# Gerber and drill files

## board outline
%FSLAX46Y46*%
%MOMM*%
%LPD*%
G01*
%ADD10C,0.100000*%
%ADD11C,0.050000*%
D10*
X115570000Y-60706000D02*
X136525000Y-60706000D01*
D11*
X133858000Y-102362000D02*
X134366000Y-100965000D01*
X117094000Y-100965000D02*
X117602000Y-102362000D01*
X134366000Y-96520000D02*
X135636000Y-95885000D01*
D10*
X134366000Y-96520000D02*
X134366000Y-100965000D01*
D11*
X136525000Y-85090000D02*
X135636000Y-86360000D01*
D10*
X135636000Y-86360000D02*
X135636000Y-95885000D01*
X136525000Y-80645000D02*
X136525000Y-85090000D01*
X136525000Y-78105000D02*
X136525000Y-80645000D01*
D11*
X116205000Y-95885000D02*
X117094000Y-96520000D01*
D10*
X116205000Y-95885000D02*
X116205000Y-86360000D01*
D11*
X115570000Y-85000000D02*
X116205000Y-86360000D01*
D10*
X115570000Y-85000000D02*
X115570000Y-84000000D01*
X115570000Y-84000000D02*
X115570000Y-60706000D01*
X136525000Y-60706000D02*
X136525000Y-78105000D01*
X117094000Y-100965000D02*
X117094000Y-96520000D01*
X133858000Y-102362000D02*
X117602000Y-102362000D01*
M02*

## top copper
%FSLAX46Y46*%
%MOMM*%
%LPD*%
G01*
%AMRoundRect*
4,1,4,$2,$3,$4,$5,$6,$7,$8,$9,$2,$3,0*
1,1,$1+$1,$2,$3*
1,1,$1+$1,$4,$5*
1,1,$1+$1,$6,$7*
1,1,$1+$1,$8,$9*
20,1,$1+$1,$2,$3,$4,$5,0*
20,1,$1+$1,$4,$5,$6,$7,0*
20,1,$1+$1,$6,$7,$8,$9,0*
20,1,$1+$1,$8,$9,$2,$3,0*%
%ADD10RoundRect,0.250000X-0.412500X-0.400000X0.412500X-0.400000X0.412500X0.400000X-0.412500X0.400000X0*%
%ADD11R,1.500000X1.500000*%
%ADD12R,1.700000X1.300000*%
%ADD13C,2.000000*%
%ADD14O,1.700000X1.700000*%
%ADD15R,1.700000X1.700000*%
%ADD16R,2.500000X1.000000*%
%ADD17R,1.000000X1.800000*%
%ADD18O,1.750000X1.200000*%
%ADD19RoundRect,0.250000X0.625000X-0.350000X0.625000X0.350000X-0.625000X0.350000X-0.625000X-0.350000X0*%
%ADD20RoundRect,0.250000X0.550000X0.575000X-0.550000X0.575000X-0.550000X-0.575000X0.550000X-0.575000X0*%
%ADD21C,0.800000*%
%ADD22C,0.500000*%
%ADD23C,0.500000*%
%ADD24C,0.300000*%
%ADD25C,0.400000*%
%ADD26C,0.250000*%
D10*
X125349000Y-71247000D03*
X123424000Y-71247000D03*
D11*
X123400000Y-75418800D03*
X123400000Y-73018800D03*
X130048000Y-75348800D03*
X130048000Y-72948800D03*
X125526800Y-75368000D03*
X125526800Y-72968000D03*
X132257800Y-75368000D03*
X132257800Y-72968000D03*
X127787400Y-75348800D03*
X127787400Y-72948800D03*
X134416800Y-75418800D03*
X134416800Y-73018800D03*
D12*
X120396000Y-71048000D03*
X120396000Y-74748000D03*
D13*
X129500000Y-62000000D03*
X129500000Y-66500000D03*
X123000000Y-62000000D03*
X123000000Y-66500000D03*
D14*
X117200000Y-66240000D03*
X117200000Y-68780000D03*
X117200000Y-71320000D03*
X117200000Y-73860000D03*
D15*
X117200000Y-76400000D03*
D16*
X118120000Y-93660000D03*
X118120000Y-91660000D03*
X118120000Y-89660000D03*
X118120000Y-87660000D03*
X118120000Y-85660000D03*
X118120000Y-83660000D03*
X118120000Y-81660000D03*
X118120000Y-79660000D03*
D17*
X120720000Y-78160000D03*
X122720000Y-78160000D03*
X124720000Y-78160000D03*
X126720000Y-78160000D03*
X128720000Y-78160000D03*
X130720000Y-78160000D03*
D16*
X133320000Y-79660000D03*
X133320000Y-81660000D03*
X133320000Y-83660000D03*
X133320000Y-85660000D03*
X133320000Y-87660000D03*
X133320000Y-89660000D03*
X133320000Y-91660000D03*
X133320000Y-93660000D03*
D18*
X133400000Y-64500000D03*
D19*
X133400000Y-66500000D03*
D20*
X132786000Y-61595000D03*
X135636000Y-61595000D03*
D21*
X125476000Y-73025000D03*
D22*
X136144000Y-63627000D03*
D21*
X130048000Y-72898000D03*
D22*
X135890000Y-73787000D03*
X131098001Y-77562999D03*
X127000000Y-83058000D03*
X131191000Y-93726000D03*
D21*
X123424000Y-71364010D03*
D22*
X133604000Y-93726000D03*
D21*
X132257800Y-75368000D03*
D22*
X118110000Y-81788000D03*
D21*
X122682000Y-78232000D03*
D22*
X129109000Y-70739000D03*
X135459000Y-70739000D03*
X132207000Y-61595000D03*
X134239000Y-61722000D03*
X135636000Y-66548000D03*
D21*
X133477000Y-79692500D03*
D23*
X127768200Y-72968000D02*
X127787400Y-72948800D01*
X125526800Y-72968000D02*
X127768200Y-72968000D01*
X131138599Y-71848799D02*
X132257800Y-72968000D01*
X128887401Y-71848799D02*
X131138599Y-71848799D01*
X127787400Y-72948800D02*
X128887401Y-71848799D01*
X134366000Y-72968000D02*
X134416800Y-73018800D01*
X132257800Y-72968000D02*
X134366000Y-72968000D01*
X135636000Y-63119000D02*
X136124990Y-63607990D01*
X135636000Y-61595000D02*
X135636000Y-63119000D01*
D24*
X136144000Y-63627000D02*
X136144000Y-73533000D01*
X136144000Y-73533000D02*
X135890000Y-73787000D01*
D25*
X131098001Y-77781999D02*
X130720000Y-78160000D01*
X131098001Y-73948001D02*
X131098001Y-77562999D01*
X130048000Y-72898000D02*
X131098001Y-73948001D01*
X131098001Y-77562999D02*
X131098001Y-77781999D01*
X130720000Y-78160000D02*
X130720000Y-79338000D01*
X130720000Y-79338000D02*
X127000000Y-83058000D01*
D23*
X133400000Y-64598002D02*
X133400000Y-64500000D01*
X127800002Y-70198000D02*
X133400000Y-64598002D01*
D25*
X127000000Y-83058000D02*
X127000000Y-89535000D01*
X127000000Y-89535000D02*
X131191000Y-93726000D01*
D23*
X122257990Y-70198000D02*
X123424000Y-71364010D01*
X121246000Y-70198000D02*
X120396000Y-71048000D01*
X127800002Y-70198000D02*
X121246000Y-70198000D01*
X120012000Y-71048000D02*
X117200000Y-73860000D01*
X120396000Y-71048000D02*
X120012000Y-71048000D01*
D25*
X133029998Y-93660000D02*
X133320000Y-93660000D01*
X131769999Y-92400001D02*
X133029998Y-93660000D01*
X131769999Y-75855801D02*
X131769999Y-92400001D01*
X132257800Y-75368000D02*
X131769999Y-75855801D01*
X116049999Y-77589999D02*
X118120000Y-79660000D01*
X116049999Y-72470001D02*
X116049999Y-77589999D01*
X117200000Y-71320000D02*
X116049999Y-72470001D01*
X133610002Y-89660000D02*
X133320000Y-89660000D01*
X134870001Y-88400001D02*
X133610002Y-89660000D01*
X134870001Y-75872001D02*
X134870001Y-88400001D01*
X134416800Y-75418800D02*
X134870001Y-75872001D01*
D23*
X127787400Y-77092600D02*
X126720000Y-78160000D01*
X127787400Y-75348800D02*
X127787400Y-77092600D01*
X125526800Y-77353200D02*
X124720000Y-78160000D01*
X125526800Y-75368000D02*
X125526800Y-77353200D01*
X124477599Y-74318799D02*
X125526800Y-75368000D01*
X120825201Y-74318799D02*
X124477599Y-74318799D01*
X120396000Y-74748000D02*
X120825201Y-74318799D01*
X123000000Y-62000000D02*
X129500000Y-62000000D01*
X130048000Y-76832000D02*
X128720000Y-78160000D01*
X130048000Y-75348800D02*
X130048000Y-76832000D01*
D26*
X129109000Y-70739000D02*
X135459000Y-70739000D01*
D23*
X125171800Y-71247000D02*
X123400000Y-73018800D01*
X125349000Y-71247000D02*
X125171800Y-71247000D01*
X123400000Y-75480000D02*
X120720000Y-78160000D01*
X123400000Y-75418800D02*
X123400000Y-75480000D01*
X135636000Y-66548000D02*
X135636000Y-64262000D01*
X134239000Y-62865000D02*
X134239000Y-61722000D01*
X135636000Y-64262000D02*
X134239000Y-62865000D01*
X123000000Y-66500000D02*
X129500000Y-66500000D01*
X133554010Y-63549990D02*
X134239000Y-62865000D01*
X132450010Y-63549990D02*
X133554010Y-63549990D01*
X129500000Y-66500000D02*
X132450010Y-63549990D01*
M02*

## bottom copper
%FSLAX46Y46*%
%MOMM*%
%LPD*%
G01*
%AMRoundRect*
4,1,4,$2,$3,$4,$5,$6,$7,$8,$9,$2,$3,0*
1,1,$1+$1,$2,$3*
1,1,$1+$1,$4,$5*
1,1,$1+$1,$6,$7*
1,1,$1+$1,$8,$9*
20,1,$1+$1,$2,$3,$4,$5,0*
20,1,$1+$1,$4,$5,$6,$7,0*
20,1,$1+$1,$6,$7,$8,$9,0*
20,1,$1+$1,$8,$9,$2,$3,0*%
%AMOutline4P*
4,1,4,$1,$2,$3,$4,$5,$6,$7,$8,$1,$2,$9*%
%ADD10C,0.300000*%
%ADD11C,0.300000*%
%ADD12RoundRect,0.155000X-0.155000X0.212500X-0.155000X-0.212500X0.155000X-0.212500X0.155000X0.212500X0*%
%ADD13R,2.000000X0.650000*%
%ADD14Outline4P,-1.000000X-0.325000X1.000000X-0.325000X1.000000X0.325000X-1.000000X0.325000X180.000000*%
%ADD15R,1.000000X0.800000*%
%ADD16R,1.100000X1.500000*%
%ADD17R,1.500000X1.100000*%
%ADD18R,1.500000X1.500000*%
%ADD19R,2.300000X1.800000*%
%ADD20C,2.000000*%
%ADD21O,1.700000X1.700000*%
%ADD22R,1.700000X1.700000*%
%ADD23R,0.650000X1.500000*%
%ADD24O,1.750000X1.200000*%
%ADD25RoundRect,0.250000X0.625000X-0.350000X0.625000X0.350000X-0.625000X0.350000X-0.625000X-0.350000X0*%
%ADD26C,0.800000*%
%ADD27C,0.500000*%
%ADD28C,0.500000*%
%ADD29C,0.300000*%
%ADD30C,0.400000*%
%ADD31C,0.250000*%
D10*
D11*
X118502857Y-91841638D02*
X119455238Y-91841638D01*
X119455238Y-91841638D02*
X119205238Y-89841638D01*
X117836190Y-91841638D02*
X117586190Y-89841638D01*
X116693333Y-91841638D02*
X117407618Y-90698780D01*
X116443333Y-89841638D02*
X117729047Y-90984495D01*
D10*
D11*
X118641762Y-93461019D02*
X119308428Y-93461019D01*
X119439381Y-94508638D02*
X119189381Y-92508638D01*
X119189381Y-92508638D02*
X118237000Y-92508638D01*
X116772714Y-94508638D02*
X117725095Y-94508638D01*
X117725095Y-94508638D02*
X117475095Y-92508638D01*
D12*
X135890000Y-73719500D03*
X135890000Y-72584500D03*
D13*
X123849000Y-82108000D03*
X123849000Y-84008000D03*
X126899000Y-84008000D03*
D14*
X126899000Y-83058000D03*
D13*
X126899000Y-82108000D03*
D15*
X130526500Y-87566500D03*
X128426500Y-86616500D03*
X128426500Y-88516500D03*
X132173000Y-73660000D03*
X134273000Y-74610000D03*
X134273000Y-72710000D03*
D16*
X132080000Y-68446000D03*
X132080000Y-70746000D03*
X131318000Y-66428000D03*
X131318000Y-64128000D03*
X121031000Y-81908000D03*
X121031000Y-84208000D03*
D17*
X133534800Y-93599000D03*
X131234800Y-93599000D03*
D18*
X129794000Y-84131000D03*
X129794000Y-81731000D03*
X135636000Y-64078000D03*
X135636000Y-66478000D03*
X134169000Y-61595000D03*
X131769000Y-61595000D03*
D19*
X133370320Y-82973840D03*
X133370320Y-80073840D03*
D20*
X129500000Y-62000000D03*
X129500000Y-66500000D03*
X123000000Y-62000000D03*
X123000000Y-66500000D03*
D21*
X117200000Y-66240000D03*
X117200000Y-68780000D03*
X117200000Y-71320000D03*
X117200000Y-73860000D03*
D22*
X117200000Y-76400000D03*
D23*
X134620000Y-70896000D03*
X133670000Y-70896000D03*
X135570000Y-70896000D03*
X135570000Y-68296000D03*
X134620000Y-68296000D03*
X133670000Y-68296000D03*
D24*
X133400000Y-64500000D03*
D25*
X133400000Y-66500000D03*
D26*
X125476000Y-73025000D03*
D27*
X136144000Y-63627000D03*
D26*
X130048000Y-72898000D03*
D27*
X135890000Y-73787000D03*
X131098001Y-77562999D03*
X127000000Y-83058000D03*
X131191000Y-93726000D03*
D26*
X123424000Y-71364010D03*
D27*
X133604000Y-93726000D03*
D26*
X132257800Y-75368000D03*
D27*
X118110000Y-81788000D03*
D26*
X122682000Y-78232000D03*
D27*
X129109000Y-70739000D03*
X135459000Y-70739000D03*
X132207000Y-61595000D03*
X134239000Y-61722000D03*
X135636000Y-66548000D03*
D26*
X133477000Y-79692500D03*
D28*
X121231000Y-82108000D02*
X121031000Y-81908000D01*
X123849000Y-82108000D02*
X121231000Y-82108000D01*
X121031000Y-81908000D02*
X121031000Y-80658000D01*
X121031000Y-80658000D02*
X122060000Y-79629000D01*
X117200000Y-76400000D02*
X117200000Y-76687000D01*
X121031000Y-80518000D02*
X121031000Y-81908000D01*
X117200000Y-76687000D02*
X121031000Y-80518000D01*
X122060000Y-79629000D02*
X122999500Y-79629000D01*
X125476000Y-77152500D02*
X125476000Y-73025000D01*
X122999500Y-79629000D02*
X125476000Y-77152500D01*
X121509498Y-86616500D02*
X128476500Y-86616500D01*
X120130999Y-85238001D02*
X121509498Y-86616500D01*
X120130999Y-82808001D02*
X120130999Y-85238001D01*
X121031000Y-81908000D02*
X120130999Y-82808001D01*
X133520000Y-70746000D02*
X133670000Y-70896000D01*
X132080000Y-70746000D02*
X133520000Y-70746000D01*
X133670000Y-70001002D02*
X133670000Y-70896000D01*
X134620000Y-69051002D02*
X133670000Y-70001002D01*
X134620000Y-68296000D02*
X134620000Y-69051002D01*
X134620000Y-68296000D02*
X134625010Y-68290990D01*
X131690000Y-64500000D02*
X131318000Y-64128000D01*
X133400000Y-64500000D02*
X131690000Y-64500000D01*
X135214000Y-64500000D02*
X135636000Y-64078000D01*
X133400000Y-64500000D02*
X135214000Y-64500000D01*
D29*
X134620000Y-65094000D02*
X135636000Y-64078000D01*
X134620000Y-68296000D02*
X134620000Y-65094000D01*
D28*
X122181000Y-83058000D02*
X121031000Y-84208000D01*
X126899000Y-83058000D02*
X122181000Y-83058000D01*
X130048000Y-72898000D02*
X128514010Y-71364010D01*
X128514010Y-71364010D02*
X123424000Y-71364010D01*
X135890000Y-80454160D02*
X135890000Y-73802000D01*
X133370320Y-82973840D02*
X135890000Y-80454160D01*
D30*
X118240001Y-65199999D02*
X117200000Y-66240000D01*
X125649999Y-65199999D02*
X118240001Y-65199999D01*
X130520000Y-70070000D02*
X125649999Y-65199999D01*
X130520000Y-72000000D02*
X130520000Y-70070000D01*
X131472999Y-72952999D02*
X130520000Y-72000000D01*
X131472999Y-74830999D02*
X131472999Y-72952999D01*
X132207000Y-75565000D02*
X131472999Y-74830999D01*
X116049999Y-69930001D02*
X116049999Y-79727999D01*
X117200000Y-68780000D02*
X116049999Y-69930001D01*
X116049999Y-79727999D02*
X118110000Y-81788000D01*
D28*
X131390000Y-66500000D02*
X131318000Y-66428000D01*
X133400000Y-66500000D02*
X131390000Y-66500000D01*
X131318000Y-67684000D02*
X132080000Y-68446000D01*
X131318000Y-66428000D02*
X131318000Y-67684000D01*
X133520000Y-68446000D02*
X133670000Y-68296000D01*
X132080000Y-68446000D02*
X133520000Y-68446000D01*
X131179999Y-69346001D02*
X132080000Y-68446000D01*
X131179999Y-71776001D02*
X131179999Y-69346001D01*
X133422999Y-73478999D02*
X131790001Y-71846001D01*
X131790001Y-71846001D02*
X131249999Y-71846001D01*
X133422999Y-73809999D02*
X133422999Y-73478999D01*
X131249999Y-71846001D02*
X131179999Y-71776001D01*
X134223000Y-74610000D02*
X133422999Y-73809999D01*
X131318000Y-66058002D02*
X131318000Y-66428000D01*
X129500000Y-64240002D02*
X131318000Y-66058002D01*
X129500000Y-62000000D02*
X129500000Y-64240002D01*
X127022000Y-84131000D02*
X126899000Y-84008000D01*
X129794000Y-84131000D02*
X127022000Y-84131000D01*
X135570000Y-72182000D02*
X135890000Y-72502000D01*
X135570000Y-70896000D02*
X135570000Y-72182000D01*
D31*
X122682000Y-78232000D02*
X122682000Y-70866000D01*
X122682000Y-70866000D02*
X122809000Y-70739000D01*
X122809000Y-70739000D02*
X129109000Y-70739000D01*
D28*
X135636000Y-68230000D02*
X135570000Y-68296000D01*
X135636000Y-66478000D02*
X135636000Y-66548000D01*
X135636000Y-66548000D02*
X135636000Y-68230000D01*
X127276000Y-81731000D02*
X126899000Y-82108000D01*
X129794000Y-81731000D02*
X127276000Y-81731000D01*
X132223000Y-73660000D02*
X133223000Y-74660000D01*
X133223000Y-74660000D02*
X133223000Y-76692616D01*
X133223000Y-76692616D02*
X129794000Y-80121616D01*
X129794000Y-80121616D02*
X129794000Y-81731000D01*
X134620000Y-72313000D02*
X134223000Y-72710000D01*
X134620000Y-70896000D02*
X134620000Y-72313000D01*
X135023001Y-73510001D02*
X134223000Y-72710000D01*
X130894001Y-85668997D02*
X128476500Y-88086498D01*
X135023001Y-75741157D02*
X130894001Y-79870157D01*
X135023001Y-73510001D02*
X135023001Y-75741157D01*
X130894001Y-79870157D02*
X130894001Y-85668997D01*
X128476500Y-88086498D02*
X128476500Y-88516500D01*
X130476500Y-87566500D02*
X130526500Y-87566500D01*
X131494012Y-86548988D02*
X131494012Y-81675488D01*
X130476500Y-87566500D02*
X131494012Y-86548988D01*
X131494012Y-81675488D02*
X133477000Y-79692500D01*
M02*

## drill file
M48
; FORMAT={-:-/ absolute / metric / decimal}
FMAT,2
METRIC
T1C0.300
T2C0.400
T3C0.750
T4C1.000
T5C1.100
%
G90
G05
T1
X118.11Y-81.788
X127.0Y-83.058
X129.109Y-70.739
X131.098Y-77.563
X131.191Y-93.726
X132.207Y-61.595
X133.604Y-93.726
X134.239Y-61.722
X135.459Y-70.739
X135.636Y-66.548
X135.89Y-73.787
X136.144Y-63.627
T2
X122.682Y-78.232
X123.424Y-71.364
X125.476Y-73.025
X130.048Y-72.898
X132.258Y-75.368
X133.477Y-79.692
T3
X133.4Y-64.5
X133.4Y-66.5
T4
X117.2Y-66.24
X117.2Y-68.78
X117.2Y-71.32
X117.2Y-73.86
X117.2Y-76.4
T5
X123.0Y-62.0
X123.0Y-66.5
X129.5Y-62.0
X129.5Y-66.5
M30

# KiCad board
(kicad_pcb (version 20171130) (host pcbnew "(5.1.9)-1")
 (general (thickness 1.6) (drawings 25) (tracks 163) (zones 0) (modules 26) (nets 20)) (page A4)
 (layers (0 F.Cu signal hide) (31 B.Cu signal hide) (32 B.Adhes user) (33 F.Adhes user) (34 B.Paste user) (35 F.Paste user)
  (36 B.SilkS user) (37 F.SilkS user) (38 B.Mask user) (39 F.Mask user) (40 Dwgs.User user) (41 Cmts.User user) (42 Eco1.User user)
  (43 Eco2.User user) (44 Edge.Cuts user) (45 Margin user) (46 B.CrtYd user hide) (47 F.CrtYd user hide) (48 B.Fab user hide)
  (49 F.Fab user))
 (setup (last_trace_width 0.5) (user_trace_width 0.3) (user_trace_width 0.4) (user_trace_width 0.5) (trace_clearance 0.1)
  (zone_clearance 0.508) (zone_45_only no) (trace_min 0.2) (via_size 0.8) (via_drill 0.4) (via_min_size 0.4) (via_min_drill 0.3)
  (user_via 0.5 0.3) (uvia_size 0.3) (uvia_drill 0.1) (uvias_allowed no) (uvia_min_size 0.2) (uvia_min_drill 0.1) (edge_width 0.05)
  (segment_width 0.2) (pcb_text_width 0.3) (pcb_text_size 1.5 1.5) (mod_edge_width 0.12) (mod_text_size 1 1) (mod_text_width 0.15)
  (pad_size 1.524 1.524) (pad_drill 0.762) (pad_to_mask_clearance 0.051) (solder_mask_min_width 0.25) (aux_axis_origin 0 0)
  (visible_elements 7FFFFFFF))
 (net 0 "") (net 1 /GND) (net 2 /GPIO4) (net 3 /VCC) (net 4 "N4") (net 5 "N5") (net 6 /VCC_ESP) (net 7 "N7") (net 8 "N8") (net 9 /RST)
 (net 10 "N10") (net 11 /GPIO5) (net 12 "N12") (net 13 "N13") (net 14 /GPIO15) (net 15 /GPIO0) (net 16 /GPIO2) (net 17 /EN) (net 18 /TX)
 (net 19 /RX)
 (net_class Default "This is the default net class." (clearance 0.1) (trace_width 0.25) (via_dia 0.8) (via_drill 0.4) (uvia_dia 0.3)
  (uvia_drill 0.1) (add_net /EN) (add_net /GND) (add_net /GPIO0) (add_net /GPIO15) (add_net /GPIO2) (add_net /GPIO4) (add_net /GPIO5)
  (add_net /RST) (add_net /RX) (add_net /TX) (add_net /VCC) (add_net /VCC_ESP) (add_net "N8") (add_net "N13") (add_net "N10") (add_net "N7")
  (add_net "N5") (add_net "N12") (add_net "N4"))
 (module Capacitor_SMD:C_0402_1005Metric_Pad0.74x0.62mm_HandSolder (layer B.Cu) (at 135.89 73.152 270)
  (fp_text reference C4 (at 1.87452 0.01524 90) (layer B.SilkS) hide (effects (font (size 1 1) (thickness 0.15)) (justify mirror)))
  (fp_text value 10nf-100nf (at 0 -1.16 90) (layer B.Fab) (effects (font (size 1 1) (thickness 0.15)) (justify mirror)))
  (pad 2 smd roundrect (at 0.5675 0 270) (size 0.735 0.62) (layers B.Cu B.Paste B.Mask) (roundrect_rratio 0.25) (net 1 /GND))
  (pad 1 smd roundrect (at -0.5675 0 270) (size 0.735 0.62) (layers B.Cu B.Paste B.Mask) (roundrect_rratio 0.25) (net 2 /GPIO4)))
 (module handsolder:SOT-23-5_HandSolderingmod (layer B.Cu) (at 125.349 83.058 180)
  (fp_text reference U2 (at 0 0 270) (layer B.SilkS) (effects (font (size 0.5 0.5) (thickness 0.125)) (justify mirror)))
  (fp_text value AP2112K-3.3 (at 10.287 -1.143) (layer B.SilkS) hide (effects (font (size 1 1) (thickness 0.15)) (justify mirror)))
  (pad 5 smd rect (at 1.5 0.95 180) (size 2 0.65) (layers B.Cu B.Paste B.Mask) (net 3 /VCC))
  (pad 4 smd rect (at 1.5 -0.95 180) (size 2 0.65) (layers B.Cu B.Paste B.Mask))
  (pad 3 smd rect (at -1.55 -0.95 180) (size 2 0.65) (layers B.Cu B.Paste B.Mask) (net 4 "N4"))
  (pad 2 smd trapezoid (at -1.55 0 180) (size 2 0.65) (layers B.Cu B.Paste B.Mask) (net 1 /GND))
  (pad 1 smd rect (at -1.55 0.95 180) (size 2 0.65) (layers B.Cu B.Paste B.Mask) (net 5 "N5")))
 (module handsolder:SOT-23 (layer B.Cu) (at 129.4765 87.5665)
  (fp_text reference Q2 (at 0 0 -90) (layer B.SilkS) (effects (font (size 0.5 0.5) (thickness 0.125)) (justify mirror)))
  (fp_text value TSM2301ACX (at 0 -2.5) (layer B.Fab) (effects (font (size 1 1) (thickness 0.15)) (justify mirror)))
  (pad 3 smd rect (at 1.05 0) (size 1 0.8) (layers B.Cu B.Paste B.Mask) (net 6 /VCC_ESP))
  (pad 2 smd rect (at -1.05 -0.95) (size 1 0.8) (layers B.Cu B.Paste B.Mask) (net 3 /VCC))
  (pad 1 smd rect (at -1.05 0.95) (size 1 0.8) (layers B.Cu B.Paste B.Mask) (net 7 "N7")))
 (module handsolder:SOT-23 (layer B.Cu) (at 133.223 73.66 180)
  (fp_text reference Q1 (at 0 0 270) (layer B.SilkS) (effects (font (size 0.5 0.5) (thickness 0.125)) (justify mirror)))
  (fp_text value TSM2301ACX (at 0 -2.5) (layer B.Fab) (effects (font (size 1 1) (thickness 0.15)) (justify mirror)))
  (pad 3 smd rect (at 1.05 0 180) (size 1 0.8) (layers B.Cu B.Paste B.Mask) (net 5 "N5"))
  (pad 2 smd rect (at -1.05 -0.95 180) (size 1 0.8) (layers B.Cu B.Paste B.Mask) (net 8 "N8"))
  (pad 1 smd rect (at -1.05 0.95 180) (size 1 0.8) (layers B.Cu B.Paste B.Mask) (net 7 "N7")))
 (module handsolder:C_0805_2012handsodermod (layer B.Cu) (at 132.08 69.596 90)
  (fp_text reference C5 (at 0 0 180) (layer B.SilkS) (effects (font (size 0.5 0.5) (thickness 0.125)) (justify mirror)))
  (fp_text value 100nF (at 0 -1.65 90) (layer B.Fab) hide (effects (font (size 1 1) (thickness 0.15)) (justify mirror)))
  (pad 2 smd rect (at 1.15 0 90) (size 1.5 1.1) (layers B.Cu B.Paste B.Mask) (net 8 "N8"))
  (pad 1 smd rect (at -1.15 0 90) (size 1.5 1.1) (layers B.Cu B.Paste B.Mask) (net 1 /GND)))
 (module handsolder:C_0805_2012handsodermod (layer B.Cu) (at 131.318 65.278 270)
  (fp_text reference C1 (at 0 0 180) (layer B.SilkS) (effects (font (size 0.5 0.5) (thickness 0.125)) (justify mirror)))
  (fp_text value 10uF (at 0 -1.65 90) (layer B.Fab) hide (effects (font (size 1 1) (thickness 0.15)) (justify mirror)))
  (pad 2 smd rect (at 1.15 0 270) (size 1.5 1.1) (layers B.Cu B.Paste B.Mask) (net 8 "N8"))
  (pad 1 smd rect (at -1.15 0 270) (size 1.5 1.1) (layers B.Cu B.Paste B.Mask) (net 1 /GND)))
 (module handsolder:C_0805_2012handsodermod (layer B.Cu) (at 121.031 83.058 90)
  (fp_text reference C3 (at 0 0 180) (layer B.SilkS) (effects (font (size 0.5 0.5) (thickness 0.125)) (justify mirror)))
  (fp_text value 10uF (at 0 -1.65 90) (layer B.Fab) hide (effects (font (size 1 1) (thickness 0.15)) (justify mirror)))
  (pad 2 smd rect (at 1.15 0 90) (size 1.5 1.1) (layers B.Cu B.Paste B.Mask) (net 3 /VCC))
  (pad 1 smd rect (at -1.15 0 90) (size 1.5 1.1) (layers B.Cu B.Paste B.Mask) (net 1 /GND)))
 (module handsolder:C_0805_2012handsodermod (layer B.Cu) (at 132.3848 93.599)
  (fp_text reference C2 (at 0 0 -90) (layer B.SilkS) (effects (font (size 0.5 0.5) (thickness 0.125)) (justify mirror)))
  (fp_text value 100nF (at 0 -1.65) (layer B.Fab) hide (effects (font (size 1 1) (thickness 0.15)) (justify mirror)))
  (pad 2 smd rect (at 1.15 0) (size 1.5 1.1) (layers B.Cu B.Paste B.Mask) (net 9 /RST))
  (pad 1 smd rect (at -1.15 0) (size 1.5 1.1) (layers B.Cu B.Paste B.Mask) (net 1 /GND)))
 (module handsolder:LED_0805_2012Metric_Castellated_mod (layer F.Cu) (at 124.3865 71.247)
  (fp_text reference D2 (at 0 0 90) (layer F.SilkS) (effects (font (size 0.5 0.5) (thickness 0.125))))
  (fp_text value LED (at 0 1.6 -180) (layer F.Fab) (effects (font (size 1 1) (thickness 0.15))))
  (pad 2 smd roundrect (at 0.9625 0) (size 1.325 1.3) (layers F.Cu F.Paste F.Mask) (roundrect_rratio 0.1923076923076923) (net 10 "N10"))
  (pad 1 smd roundrect (at -0.9625 0) (size 1.325 1.3) (layers F.Cu F.Paste F.Mask) (roundrect_rratio 0.1923076923076923) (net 1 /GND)))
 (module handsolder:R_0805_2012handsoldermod (layer F.Cu) (at 123.4 74.2188 270)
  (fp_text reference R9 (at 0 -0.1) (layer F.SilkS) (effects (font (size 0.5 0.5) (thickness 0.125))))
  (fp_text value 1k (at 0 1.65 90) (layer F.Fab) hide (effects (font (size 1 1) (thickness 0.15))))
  (pad 2 smd rect (at 1.2 0 270) (size 1.5 1.5) (layers F.Cu F.Paste F.Mask) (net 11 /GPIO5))
  (pad 1 smd rect (at -1.2 0 270) (size 1.5 1.5) (layers F.Cu F.Paste F.Mask) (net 10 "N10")))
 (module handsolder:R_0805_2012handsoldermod (layer B.Cu) (at 129.794 82.931 270)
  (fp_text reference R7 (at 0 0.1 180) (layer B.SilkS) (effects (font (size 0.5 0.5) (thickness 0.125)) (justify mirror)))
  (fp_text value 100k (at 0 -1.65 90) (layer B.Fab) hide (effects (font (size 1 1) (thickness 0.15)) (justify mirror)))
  (pad 2 smd rect (at 1.2 0 270) (size 1.5 1.5) (layers B.Cu B.Paste B.Mask) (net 4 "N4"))
  (pad 1 smd rect (at -1.2 0 270) (size 1.5 1.5) (layers B.Cu B.Paste B.Mask) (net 5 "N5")))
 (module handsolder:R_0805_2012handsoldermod (layer B.Cu) (at 135.636 65.278 90)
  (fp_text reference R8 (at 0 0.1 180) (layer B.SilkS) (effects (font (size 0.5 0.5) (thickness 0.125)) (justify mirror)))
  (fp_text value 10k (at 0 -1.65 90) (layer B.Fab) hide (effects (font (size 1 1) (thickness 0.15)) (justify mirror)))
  (pad 2 smd rect (at 1.2 0 90) (size 1.5 1.5) (layers B.Cu B.Paste B.Mask) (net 1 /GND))
  (pad 1 smd rect (at -1.2 0 90) (size 1.5 1.5) (layers B.Cu B.Paste B.Mask) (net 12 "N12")))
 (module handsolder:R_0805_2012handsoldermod (layer B.Cu) (at 132.969 61.595)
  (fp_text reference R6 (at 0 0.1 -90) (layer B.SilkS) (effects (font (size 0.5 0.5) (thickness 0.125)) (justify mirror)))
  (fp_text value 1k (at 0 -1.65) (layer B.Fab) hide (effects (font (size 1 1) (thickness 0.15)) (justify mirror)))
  (pad 2 smd rect (at 1.2 0) (size 1.5 1.5) (layers B.Cu B.Paste B.Mask) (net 12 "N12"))
  (pad 1 smd rect (at -1.2 0) (size 1.5 1.5) (layers B.Cu B.Paste B.Mask) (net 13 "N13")))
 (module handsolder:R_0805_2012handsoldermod (layer F.Cu) (at 130.048 74.1488 270)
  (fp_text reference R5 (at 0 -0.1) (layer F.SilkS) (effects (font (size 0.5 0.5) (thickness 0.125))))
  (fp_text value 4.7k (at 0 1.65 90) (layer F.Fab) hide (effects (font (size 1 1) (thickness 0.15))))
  (pad 2 smd rect (at 1.2 0 270) (size 1.5 1.5) (layers F.Cu F.Paste F.Mask) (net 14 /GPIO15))
  (pad 1 smd rect (at -1.2 0 270) (size 1.5 1.5) (layers F.Cu F.Paste F.Mask) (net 1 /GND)))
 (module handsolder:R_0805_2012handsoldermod (layer F.Cu) (at 125.5268 74.168 270)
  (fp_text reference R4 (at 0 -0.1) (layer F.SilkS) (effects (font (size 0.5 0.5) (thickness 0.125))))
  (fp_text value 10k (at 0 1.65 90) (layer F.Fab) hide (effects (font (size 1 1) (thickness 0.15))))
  (pad 2 smd rect (at 1.2 0 270) (size 1.5 1.5) (layers F.Cu F.Paste F.Mask) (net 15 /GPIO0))
  (pad 1 smd rect (at -1.2 0 270) (size 1.5 1.5) (layers F.Cu F.Paste F.Mask) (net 3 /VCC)))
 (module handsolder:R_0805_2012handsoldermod (layer F.Cu) (at 132.2578 74.168 270)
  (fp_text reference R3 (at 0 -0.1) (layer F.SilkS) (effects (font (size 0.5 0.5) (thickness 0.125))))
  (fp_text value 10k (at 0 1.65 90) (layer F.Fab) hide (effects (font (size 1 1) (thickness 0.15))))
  (pad 2 smd rect (at 1.2 0 270) (size 1.5 1.5) (layers F.Cu F.Paste F.Mask) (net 9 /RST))
  (pad 1 smd rect (at -1.2 0 270) (size 1.5 1.5) (layers F.Cu F.Paste F.Mask) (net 3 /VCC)))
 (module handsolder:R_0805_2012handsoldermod (layer F.Cu) (at 127.7874 74.1488 270)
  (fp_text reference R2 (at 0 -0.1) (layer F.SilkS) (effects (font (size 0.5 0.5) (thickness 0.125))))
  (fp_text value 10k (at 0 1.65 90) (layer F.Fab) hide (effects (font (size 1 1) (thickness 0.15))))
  (pad 2 smd rect (at 1.2 0 270) (size 1.5 1.5) (layers F.Cu F.Paste F.Mask) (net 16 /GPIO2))
  (pad 1 smd rect (at -1.2 0 270) (size 1.5 1.5) (layers F.Cu F.Paste F.Mask) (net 3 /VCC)))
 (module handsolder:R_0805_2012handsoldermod (layer F.Cu) (at 134.4168 74.2188 270)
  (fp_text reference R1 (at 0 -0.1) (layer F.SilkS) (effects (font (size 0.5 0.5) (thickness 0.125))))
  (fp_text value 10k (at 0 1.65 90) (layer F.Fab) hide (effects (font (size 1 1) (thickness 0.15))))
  (pad 2 smd rect (at 1.2 0 270) (size 1.5 1.5) (layers F.Cu F.Paste F.Mask) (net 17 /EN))
  (pad 1 smd rect (at -1.2 0 270) (size 1.5 1.5) (layers F.Cu F.Paste F.Mask) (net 3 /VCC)))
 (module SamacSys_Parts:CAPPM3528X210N (layer B.Cu) (at 133.37032 81.52384 270)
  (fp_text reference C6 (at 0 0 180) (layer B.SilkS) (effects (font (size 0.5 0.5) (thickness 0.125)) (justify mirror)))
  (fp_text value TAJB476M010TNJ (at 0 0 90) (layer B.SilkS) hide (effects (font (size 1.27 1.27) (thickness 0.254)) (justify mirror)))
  (pad 2 smd rect (at 1.45 0 270) (size 1.8 2.3) (layers B.Cu B.Paste B.Mask) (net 1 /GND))
  (pad 1 smd rect (at -1.45 0 270) (size 1.8 2.3) (layers B.Cu B.Paste B.Mask) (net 6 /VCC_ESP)))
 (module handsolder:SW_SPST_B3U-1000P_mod (layer F.Cu) (at 120.396 72.898 90)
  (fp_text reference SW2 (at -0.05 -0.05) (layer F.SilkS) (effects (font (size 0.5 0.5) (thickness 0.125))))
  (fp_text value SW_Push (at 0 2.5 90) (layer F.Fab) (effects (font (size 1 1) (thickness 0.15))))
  (pad 2 smd rect (at 1.85 0 90) (size 1.3 1.7) (layers F.Cu F.Paste F.Mask) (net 1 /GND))
  (pad 1 smd rect (at -1.85 0 90) (size 1.3 1.7) (layers F.Cu F.Paste F.Mask) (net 15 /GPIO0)))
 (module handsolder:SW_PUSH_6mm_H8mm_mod (layer F.Cu) (at 123 62)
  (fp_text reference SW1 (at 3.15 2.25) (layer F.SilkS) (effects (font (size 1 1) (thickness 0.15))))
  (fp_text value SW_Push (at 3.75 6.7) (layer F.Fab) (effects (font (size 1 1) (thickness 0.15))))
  (pad 1 thru_hole circle (at 6.5 0 90) (size 2 2) (drill 1.1) (layers *.Cu *.Mask) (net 8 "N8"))
  (pad 2 thru_hole circle (at 6.5 4.5 90) (size 2 2) (drill 1.1) (layers *.Cu *.Mask) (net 12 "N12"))
  (pad 1 thru_hole circle (at 0 0 90) (size 2 2) (drill 1.1) (layers *.Cu *.Mask) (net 8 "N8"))
  (pad 2 thru_hole circle (at 0 4.5 90) (size 2 2) (drill 1.1) (layers *.Cu *.Mask) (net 12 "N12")))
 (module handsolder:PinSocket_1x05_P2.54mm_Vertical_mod (layer F.Cu) (at 117.2 76.4 180)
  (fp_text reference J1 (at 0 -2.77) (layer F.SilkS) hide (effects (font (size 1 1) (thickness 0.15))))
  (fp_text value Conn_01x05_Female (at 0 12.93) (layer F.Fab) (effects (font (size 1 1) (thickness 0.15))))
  (pad 5 thru_hole oval (at 0 10.16 180) (size 1.7 1.7) (drill 1) (layers *.Cu *.Mask) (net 9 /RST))
  (pad 4 thru_hole oval (at 0 7.62 180) (size 1.7 1.7) (drill 1) (layers *.Cu *.Mask) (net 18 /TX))
  (pad 3 thru_hole oval (at 0 5.08 180) (size 1.7 1.7) (drill 1) (layers *.Cu *.Mask) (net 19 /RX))
  (pad 2 thru_hole oval (at 0 2.54 180) (size 1.7 1.7) (drill 1) (layers *.Cu *.Mask) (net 1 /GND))
  (pad 1 thru_hole rect (at 0 0 180) (size 1.7 1.7) (drill 1) (layers *.Cu *.Mask) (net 3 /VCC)))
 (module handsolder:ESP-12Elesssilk (layer F.Cu) (at 125.72 90.16 180)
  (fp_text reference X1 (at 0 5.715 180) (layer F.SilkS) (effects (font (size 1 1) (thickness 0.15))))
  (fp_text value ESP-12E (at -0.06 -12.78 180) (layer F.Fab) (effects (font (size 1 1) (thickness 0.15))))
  (pad 22 smd rect (at 7.6 -3.5 180) (size 2.5 1) (layers F.Cu F.Paste F.Mask))
  (pad 21 smd rect (at 7.6 -1.5 180) (size 2.5 1) (layers F.Cu F.Paste F.Mask))
  (pad 20 smd rect (at 7.6 0.5 180) (size 2.5 1) (layers F.Cu F.Paste F.Mask))
  (pad 19 smd rect (at 7.6 2.5 180) (size 2.5 1) (layers F.Cu F.Paste F.Mask))
  (pad 18 smd rect (at 7.6 4.5 180) (size 2.5 1) (layers F.Cu F.Paste F.Mask))
  (pad 17 smd rect (at 7.6 6.5 180) (size 2.5 1) (layers F.Cu F.Paste F.Mask))
  (pad 16 smd rect (at 7.6 8.5 180) (size 2.5 1) (layers F.Cu F.Paste F.Mask) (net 18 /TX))
  (pad 15 smd rect (at 7.6 10.5 180) (size 2.5 1) (layers F.Cu F.Paste F.Mask) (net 19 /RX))
  (pad 14 smd rect (at 5 12 180) (size 1 1.8) (layers F.Cu F.Paste F.Mask) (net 11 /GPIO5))
  (pad 13 smd rect (at 3 12 180) (size 1 1.8) (layers F.Cu F.Paste F.Mask) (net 2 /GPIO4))
  (pad 12 smd rect (at 1 12 180) (size 1 1.8) (layers F.Cu F.Paste F.Mask) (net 15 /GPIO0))
  (pad 11 smd rect (at -1 12 180) (size 1 1.8) (layers F.Cu F.Paste F.Mask) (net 16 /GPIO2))
  (pad 10 smd rect (at -3 12 180) (size 1 1.8) (layers F.Cu F.Paste F.Mask) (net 14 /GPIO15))
  (pad 9 smd rect (at -5 12 180) (size 1 1.8) (layers F.Cu F.Paste F.Mask) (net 1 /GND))
  (pad 8 smd rect (at -7.6 10.5 180) (size 2.5 1) (layers F.Cu F.Paste F.Mask) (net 6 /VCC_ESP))
  (pad 7 smd rect (at -7.6 8.5 180) (size 2.5 1) (layers F.Cu F.Paste F.Mask))
  (pad 6 smd rect (at -7.6 6.5 180) (size 2.5 1) (layers F.Cu F.Paste F.Mask))
  (pad 5 smd rect (at -7.6 4.5 180) (size 2.5 1) (layers F.Cu F.Paste F.Mask))
  (pad 4 smd rect (at -7.6 2.5 180) (size 2.5 1) (layers F.Cu F.Paste F.Mask))
  (pad 3 smd rect (at -7.6 0.5 180) (size 2.5 1) (layers F.Cu F.Paste F.Mask) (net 17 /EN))
  (pad 2 smd rect (at -7.6 -1.5 180) (size 2.5 1) (layers F.Cu F.Paste F.Mask))
  (pad 1 smd rect (at -7.6 -3.5 180) (size 2.5 1) (layers F.Cu F.Paste F.Mask) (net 9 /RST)))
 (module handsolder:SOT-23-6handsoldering (layer B.Cu) (at 134.62 69.596 270)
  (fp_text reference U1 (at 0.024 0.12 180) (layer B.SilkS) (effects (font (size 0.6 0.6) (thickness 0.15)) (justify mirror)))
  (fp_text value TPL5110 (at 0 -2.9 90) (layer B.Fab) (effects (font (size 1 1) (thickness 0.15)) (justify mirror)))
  (pad 5 smd rect (at 1.3 0 270) (size 1.5 0.65) (layers B.Cu B.Paste B.Mask) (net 7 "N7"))
  (pad 6 smd rect (at 1.3 0.95 270) (size 1.5 0.65) (layers B.Cu B.Paste B.Mask) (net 1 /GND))
  (pad 4 smd rect (at 1.3 -0.95 270) (size 1.5 0.65) (layers B.Cu B.Paste B.Mask) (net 2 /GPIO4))
  (pad 3 smd rect (at -1.3 -0.95 270) (size 1.5 0.65) (layers B.Cu B.Paste B.Mask) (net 12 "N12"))
  (pad 2 smd rect (at -1.3 0 270) (size 1.5 0.65) (layers B.Cu B.Paste B.Mask) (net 1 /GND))
  (pad 1 smd rect (at -1.3 0.95 270) (size 1.5 0.65) (layers B.Cu B.Paste B.Mask) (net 8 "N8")))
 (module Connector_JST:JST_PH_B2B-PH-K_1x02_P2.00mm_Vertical (layer F.Cu) (at 133.4 66.5 90)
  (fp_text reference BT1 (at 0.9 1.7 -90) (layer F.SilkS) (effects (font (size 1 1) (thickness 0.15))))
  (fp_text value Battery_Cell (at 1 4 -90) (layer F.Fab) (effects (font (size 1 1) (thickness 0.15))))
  (pad 2 thru_hole oval (at 2 0 90) (size 1.2 1.75) (drill 0.75) (layers *.Cu *.Mask) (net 1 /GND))
  (pad 1 thru_hole roundrect (at 0 0 90) (size 1.2 1.75) (drill 0.75) (layers *.Cu *.Mask) (roundrect_rratio 0.208333) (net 8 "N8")))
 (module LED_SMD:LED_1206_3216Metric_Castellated (layer F.Cu) (at 134.211 61.595 180)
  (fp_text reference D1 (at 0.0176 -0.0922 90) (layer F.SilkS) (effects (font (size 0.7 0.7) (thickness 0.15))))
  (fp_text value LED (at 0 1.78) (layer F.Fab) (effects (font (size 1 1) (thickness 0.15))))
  (pad 2 smd roundrect (at 1.425 0 180) (size 1.6 1.65) (layers F.Cu F.Paste F.Mask) (roundrect_rratio 0.15625) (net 13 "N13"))
  (pad 1 smd roundrect (at -1.425 0 180) (size 1.6 1.65) (layers F.Cu F.Paste F.Mask) (roundrect_rratio 0.15625) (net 1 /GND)))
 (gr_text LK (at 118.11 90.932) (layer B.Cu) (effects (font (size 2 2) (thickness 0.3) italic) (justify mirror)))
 (gr_line (start 115.57 60.706) (end 136.525 60.706) (layer Edge.Cuts) (width 0.1))
 (gr_line (start 133.858 102.362) (end 134.366 100.965) (layer Edge.Cuts) (width 0.05))
 (gr_line (start 117.094 100.965) (end 117.602 102.362) (layer Edge.Cuts) (width 0.05))
 (gr_line (start 134.366 96.52) (end 135.636 95.885) (layer Edge.Cuts) (width 0.05))
 (gr_line (start 134.366 96.52) (end 134.366 100.965) (layer Edge.Cuts) (width 0.1))
 (gr_line (start 136.525 85.09) (end 135.636 86.36) (layer Edge.Cuts) (width 0.05))
 (gr_line (start 135.636 86.36) (end 135.636 95.885) (layer Edge.Cuts) (width 0.1))
 (gr_line (start 136.525 80.645) (end 136.525 85.09) (layer Edge.Cuts) (width 0.1))
 (gr_line (start 136.525 78.105) (end 136.525 80.645) (layer Edge.Cuts) (width 0.1))
 (gr_line (start 116.205 95.885) (end 117.094 96.52) (layer Edge.Cuts) (width 0.05))
 (gr_line (start 116.205 95.885) (end 116.205 86.36) (layer Edge.Cuts) (width 0.1))
 (gr_line (start 115.57 85) (end 116.205 86.36) (layer Edge.Cuts) (width 0.05))
 (gr_line (start 115.57 85) (end 115.57 84) (layer Edge.Cuts) (width 0.1))
 (gr_line (start 115.57 84) (end 115.57 60.706) (layer Edge.Cuts) (width 0.1))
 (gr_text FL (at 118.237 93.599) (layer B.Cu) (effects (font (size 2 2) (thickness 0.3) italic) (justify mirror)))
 (gr_line (start 136.525 60.706) (end 136.525 78.105) (layer Edge.Cuts) (width 0.1))
 (gr_line (start 117.094 100.965) (end 117.094 96.52) (layer Edge.Cuts) (width 0.1))
 (gr_line (start 133.858 102.362) (end 117.602 102.362) (layer Edge.Cuts) (width 0.1))
 (via (at 125.476 73.025) (size 0.8) (drill 0.4) (layers F.Cu B.Cu) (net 3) (status 30))
 (segment (start 121.231 82.108) (end 121.031 81.908) (width 0.5) (layer B.Cu) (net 3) (status 30))
 (segment (start 123.849 82.108) (end 121.231 82.108) (width 0.5) (layer B.Cu) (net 3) (status 30))
 (segment (start 121.031 81.908) (end 121.031 80.658) (width 0.5) (layer B.Cu) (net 3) (status 10))
 (segment (start 121.031 80.658) (end 122.06 79.629) (width 0.5) (layer B.Cu) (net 3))
 (segment (start 127.7682 72.968) (end 127.7874 72.9488) (width 0.5) (layer F.Cu) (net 3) (status 30))
 (segment (start 125.5268 72.968) (end 127.7682 72.968) (width 0.5) (layer F.Cu) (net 3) (status 30))
 (segment (start 131.138599 71.848799) (end 132.2578 72.968) (width 0.5) (layer F.Cu) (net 3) (status 20))
 (segment (start 128.887401 71.848799) (end 131.138599 71.848799) (width 0.5) (layer F.Cu) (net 3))
 (segment (start 127.7874 72.9488) (end 128.887401 71.848799) (width 0.5) (layer F.Cu) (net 3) (status 10))
 (segment (start 134.366 72.968) (end 134.4168 73.0188) (width 0.5) (layer F.Cu) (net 3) (status 30))
 (segment (start 132.2578 72.968) (end 134.366 72.968) (width 0.5) (layer F.Cu) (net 3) (status 30))
 (segment (start 117.2 76.4) (end 117.2 76.687) (width 0.5) (layer B.Cu) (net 3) (status 30))
 (segment (start 121.031 80.518) (end 121.031 81.908) (width 0.5) (layer B.Cu) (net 3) (status 20))
 (segment (start 117.2 76.687) (end 121.031 80.518) (width 0.5) (layer B.Cu) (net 3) (status 10))
 (segment (start 122.06 79.629) (end 122.9995 79.629) (width 0.5) (layer B.Cu) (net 3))
 (segment (start 125.476 77.1525) (end 125.476 73.025) (width 0.5) (layer B.Cu) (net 3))
 (segment (start 122.9995 79.629) (end 125.476 77.1525) (width 0.5) (layer B.Cu) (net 3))
 (segment (start 121.509498 86.6165) (end 128.4765 86.6165) (width 0.5) (layer B.Cu) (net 3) (status 20))
 (segment (start 120.130999 85.238001) (end 121.509498 86.6165) (width 0.5) (layer B.Cu) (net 3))
 (segment (start 120.130999 82.808001) (end 120.130999 85.238001) (width 0.5) (layer B.Cu) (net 3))
 (segment (start 121.031 81.908) (end 120.130999 82.808001) (width 0.5) (layer B.Cu) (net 3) (status 10))
 (via (at 136.144 63.627) (size 0.5) (drill 0.3) (layers F.Cu B.Cu) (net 1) (status 30))
 (segment (start 133.52 70.746) (end 133.67 70.896) (width 0.5) (layer B.Cu) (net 1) (status 30))
 (segment (start 132.08 70.746) (end 133.52 70.746) (width 0.5) (layer B.Cu) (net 1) (status 30))
 (segment (start 133.67 70.001002) (end 133.67 70.896) (width 0.5) (layer B.Cu) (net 1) (status 20))
 (segment (start 134.62 69.051002) (end 133.67 70.001002) (width 0.5) (layer B.Cu) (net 1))
 (segment (start 134.62 68.296) (end 134.62 69.051002) (width 0.5) (layer B.Cu) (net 1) (status 10))
 (segment (start 134.62 68.296) (end 134.62501 68.29099) (width 0.5) (layer B.Cu) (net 1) (status 30))
 (segment (start 131.69 64.5) (end 131.318 64.128) (width 0.5) (layer B.Cu) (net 1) (status 30))
 (segment (start 133.4 64.5) (end 131.69 64.5) (width 0.5) (layer B.Cu) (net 1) (status 30))
 (segment (start 135.214 64.5) (end 135.636 64.078) (width 0.5) (layer B.Cu) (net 1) (status 30))
 (segment (start 133.4 64.5) (end 135.214 64.5) (width 0.5) (layer B.Cu) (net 1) (status 30))
 (segment (start 134.62 65.094) (end 135.636 64.078) (width 0.3) (layer B.Cu) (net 1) (status 20))
 (segment (start 134.62 68.296) (end 134.62 65.094) (width 0.3) (layer B.Cu) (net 1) (status 10))
 (segment (start 122.181 83.058) (end 121.031 84.208) (width 0.5) (layer B.Cu) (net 1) (status 20))
 (segment (start 126.899 83.058) (end 122.181 83.058) (width 0.5) (layer B.Cu) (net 1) (status 10))
 (segment (start 135.636 63.119) (end 136.12499 63.60799) (width 0.5) (layer F.Cu) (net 1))
 (segment (start 135.636 61.595) (end 135.636 63.119) (width 0.5) (layer F.Cu) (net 1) (status 10))
 (via (at 130.048 72.898) (size 0.8) (drill 0.4) (layers F.Cu B.Cu) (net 1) (status 30))
 (segment (start 136.144 63.627) (end 136.144 73.533) (width 0.3) (layer F.Cu) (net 1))
 (segment (start 136.144 73.533) (end 135.89 73.787) (width 0.3) (layer F.Cu) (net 1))
 (via (at 135.89 73.787) (size 0.5) (drill 0.3) (layers F.Cu B.Cu) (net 1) (status 30))
 (segment (start 131.098001 77.781999) (end 130.72 78.16) (width 0.4) (layer F.Cu) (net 1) (status 30))
 (segment (start 131.098001 73.948001) (end 131.098001 77.562999) (width 0.4) (layer F.Cu) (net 1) (status 20))
 (segment (start 130.048 72.898) (end 131.098001 73.948001) (width 0.4) (layer F.Cu) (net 1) (status 10))
 (segment (start 131.098001 77.562999) (end 131.098001 77.781999) (width 0.4) (layer F.Cu) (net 1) (status 30))
 (via (at 131.098001 77.562999) (size 0.5) (drill 0.3) (layers F.Cu B.Cu) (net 1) (status 30))
 (segment (start 130.72 78.16) (end 130.72 79.338) (width 0.4) (layer F.Cu) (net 1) (status 10))
 (segment (start 130.72 79.338) (end 127 83.058) (width 0.4) (layer F.Cu) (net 1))
 (via (at 127 83.058) (size 0.5) (drill 0.3) (layers F.Cu B.Cu) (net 1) (status 30))
 (segment (start 133.4 64.598002) (end 133.4 64.5) (width 0.5) (layer F.Cu) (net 1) (status 30))
 (segment (start 127.800002 70.198) (end 133.4 64.598002) (width 0.5) (layer F.Cu) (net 1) (status 20))
 (via (at 131.191 93.726) (size 0.5) (drill 0.3) (layers F.Cu B.Cu) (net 1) (status 30))
 (segment (start 127 83.058) (end 127 89.535) (width 0.4) (layer F.Cu) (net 1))
 (segment (start 127 89.535) (end 131.191 93.726) (width 0.4) (layer F.Cu) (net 1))
 (via (at 123.424 71.36401) (size 0.8) (drill 0.4) (layers F.Cu B.Cu) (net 1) (status 30))
 (segment (start 122.25799 70.198) (end 123.424 71.36401) (width 0.5) (layer F.Cu) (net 1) (status 20))
 (segment (start 130.048 72.898) (end 128.51401 71.36401) (width 0.5) (layer B.Cu) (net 1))
 (segment (start 128.51401 71.36401) (end 123.424 71.36401) (width 0.5) (layer B.Cu) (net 1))
 (segment (start 121.246 70.198) (end 120.396 71.048) (width 0.5) (layer F.Cu) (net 1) (status 20))
 (segment (start 127.800002 70.198) (end 121.246 70.198) (width 0.5) (layer F.Cu) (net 1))
 (segment (start 120.012 71.048) (end 117.2 73.86) (width 0.5) (layer F.Cu) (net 1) (status 30))
 (segment (start 120.396 71.048) (end 120.012 71.048) (width 0.5) (layer F.Cu) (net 1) (status 30))
 (segment (start 135.89 80.45416) (end 135.89 73.802) (width 0.5) (layer B.Cu) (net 1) (status 20))
 (segment (start 133.37032 82.97384) (end 135.89 80.45416) (width 0.5) (layer B.Cu) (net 1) (status 10))
 (via (at 133.604 93.726) (size 0.5) (drill 0.3) (layers F.Cu B.Cu) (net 9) (status 30))
 (segment (start 133.029998 93.66) (end 133.32 93.66) (width 0.4) (layer F.Cu) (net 9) (status 30))
 (segment (start 131.769999 92.400001) (end 133.029998 93.66) (width 0.4) (layer F.Cu) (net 9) (status 20))
 (segment (start 131.769999 75.855801) (end 131.769999 92.400001) (width 0.4) (layer F.Cu) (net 9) (status 10))
 (segment (start 132.2578 75.368) (end 131.769999 75.855801) (width 0.4) (layer F.Cu) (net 9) (status 30))
 (via (at 132.2578 75.368) (size 0.8) (drill 0.4) (layers F.Cu B.Cu) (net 9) (status 30))
 (segment (start 118.240001 65.199999) (end 117.2 66.24) (width 0.4) (layer B.Cu) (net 9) (status 20))
 (segment (start 125.649999 65.199999) (end 118.240001 65.199999) (width 0.4) (layer B.Cu) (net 9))
 (segment (start 130.52 70.07) (end 125.649999 65.199999) (width 0.4) (layer B.Cu) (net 9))
 (segment (start 130.52 72) (end 130.52 70.07) (width 0.4) (layer B.Cu) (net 9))
 (segment (start 131.472999 72.952999) (end 130.52 72) (width 0.4) (layer B.Cu) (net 9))
 (segment (start 131.472999 74.830999) (end 131.472999 72.952999) (width 0.4) (layer B.Cu) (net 9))
 (segment (start 132.207 75.565) (end 131.472999 74.830999) (width 0.4) (layer B.Cu) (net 9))
 (segment (start 116.049999 77.589999) (end 118.12 79.66) (width 0.4) (layer F.Cu) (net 19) (status 20))
 (segment (start 116.049999 72.470001) (end 116.049999 77.589999) (width 0.4) (layer F.Cu) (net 19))
 (segment (start 117.2 71.32) (end 116.049999 72.470001) (width 0.4) (layer F.Cu) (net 19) (status 10))
 (segment (start 116.049999 69.930001) (end 116.049999 79.727999) (width 0.4) (layer B.Cu) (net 18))
 (segment (start 117.2 68.78) (end 116.049999 69.930001) (width 0.4) (layer B.Cu) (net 18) (status 10))
 (segment (start 116.049999 79.727999) (end 118.11 81.788) (width 0.4) (layer B.Cu) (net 18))
 (via (at 118.11 81.788) (size 0.5) (drill 0.3) (layers F.Cu B.Cu) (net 18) (status 30))
 (segment (start 133.610002 89.66) (end 133.32 89.66) (width 0.4) (layer F.Cu) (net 17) (status 30))
 (segment (start 134.870001 88.400001) (end 133.610002 89.66) (width 0.4) (layer F.Cu) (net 17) (status 20))
 (segment (start 134.870001 75.872001) (end 134.870001 88.400001) (width 0.4) (layer F.Cu) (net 17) (status 10))
 (segment (start 134.4168 75.4188) (end 134.870001 75.872001) (width 0.4) (layer F.Cu) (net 17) (status 30))
 (segment (start 127.7874 77.0926) (end 126.72 78.16) (width 0.5) (layer F.Cu) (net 16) (status 20))
 (segment (start 127.7874 75.3488) (end 127.7874 77.0926) (width 0.5) (layer F.Cu) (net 16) (status 10))
 (segment (start 125.5268 77.3532) (end 124.72 78.16) (width 0.5) (layer F.Cu) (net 15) (status 20))
 (segment (start 125.5268 75.368) (end 125.5268 77.3532) (width 0.5) (layer F.Cu) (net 15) (status 10))
 (segment (start 124.477599 74.318799) (end 125.5268 75.368) (width 0.5) (layer F.Cu) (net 15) (status 20))
 (segment (start 120.825201 74.318799) (end 124.477599 74.318799) (width 0.5) (layer F.Cu) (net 15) (status 10))
 (segment (start 120.396 74.748) (end 120.825201 74.318799) (width 0.5) (layer F.Cu) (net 15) (status 30))
 (segment (start 131.39 66.5) (end 131.318 66.428) (width 0.5) (layer B.Cu) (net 8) (status 30))
 (segment (start 133.4 66.5) (end 131.39 66.5) (width 0.5) (layer B.Cu) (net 8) (status 30))
 (segment (start 131.318 67.684) (end 132.08 68.446) (width 0.5) (layer B.Cu) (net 8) (status 20))
 (segment (start 131.318 66.428) (end 131.318 67.684) (width 0.5) (layer B.Cu) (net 8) (status 10))
 (segment (start 133.52 68.446) (end 133.67 68.296) (width 0.5) (layer B.Cu) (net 8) (status 30))
 (segment (start 132.08 68.446) (end 133.52 68.446) (width 0.5) (layer B.Cu) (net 8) (status 30))
 (segment (start 131.179999 69.346001) (end 132.08 68.446) (width 0.5) (layer B.Cu) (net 8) (status 20))
 (segment (start 131.179999 71.776001) (end 131.179999 69.346001) (width 0.5) (layer B.Cu) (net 8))
 (segment (start 133.422999 73.478999) (end 131.790001 71.846001) (width 0.5) (layer B.Cu) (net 8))
 (segment (start 131.790001 71.846001) (end 131.249999 71.846001) (width 0.5) (layer B.Cu) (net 8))
 (segment (start 133.422999 73.809999) (end 133.422999 73.478999) (width 0.5) (layer B.Cu) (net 8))
 (segment (start 131.249999 71.846001) (end 131.179999 71.776001) (width 0.5) (layer B.Cu) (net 8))
 (segment (start 134.223 74.61) (end 133.422999 73.809999) (width 0.5) (layer B.Cu) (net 8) (status 10))
 (segment (start 123 62) (end 129.5 62) (width 0.5) (layer F.Cu) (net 8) (status 30))
 (segment (start 131.318 66.058002) (end 131.318 66.428) (width 0.5) (layer B.Cu) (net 8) (status 30))
 (segment (start 129.5 64.240002) (end 131.318 66.058002) (width 0.5) (layer B.Cu) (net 8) (status 20))
 (segment (start 129.5 62) (end 129.5 64.240002) (width 0.5) (layer B.Cu) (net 8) (status 10))
 (segment (start 130.048 76.832) (end 128.72 78.16) (width 0.5) (layer F.Cu) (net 14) (status 20))
 (segment (start 130.048 75.3488) (end 130.048 76.832) (width 0.5) (layer F.Cu) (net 14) (status 10))
 (segment (start 127.022 84.131) (end 126.899 84.008) (width 0.5) (layer B.Cu) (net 4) (status 30))
 (segment (start 129.794 84.131) (end 127.022 84.131) (width 0.5) (layer B.Cu) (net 4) (status 30))
 (via (at 122.682 78.232) (size 0.8) (drill 0.4) (layers F.Cu B.Cu) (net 2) (status 30))
 (segment (start 135.57 72.182) (end 135.89 72.502) (width 0.5) (layer B.Cu) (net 2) (status 20))
 (segment (start 135.57 70.896) (end 135.57 72.182) (width 0.5) (layer B.Cu) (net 2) (status 10))
 (segment (start 122.682 78.232) (end 122.682 70.866) (width 0.25) (layer B.Cu) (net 2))
 (segment (start 122.682 70.866) (end 122.809 70.739) (width 0.25) (layer B.Cu) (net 2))
 (segment (start 122.809 70.739) (end 129.109 70.739) (width 0.25) (layer B.Cu) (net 2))
 (via (at 129.109 70.739) (size 0.5) (drill 0.3) (layers F.Cu B.Cu) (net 2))
 (segment (start 129.109 70.739) (end 135.459 70.739) (width 0.25) (layer F.Cu) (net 2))
 (via (at 135.459 70.739) (size 0.5) (drill 0.3) (layers F.Cu B.Cu) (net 2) (status 30))
 (segment (start 125.1718 71.247) (end 123.4 73.0188) (width 0.5) (layer F.Cu) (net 10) (status 30))
 (segment (start 125.349 71.247) (end 125.1718 71.247) (width 0.5) (layer F.Cu) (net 10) (status 30))
 (segment (start 123.4 75.48) (end 120.72 78.16) (width 0.5) (layer F.Cu) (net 11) (status 30))
 (segment (start 123.4 75.4188) (end 123.4 75.48) (width 0.5) (layer F.Cu) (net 11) (status 30))
 (via (at 132.207 61.595) (size 0.5) (drill 0.3) (layers F.Cu B.Cu) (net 13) (status 30))
 (via (at 134.239 61.722) (size 0.5) (drill 0.3) (layers F.Cu B.Cu) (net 12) (status 30))
 (segment (start 135.636 68.23) (end 135.57 68.296) (width 0.5) (layer B.Cu) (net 12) (status 30))
 (segment (start 135.636 66.478) (end 135.636 66.548) (width 0.5) (layer B.Cu) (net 12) (status 30))
 (segment (start 135.636 66.548) (end 135.636 68.23) (width 0.5) (layer B.Cu) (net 12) (status 30))
 (via (at 135.636 66.548) (size 0.5) (drill 0.3) (layers F.Cu B.Cu) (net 12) (status 30))
 (segment (start 135.636 66.548) (end 135.636 64.262) (width 0.5) (layer F.Cu) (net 12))
 (segment (start 134.239 62.865) (end 134.239 61.722) (width 0.5) (layer F.Cu) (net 12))
 (segment (start 135.636 64.262) (end 134.239 62.865) (width 0.5) (layer F.Cu) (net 12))
 (segment (start 123 66.5) (end 129.5 66.5) (width 0.5) (layer F.Cu) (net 12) (status 30))
 (segment (start 133.55401 63.54999) (end 134.239 62.865) (width 0.5) (layer F.Cu) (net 12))
 (segment (start 132.45001 63.54999) (end 133.55401 63.54999) (width 0.5) (layer F.Cu) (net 12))
 (segment (start 129.5 66.5) (end 132.45001 63.54999) (width 0.5) (layer F.Cu) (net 12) (status 10))
 (segment (start 127.276 81.731) (end 126.899 82.108) (width 0.5) (layer B.Cu) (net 5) (status 20))
 (segment (start 129.794 81.731) (end 127.276 81.731) (width 0.5) (layer B.Cu) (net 5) (status 10))
 (segment (start 132.223 73.66) (end 133.223 74.66) (width 0.5) (layer B.Cu) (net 5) (status 10))
 (segment (start 133.223 74.66) (end 133.223 76.692616) (width 0.5) (layer B.Cu) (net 5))
 (segment (start 133.223 76.692616) (end 129.794 80.121616) (width 0.5) (layer B.Cu) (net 5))
 (segment (start 129.794 80.121616) (end 129.794 81.731) (width 0.5) (layer B.Cu) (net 5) (status 20))
 (segment (start 134.62 72.313) (end 134.223 72.71) (width 0.5) (layer B.Cu) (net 7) (status 30))
 (segment (start 134.62 70.896) (end 134.62 72.313) (width 0.5) (layer B.Cu) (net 7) (status 30))
 (segment (start 135.023001 73.510001) (end 134.223 72.71) (width 0.5) (layer B.Cu) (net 7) (status 20))
 (segment (start 130.894001 85.668997) (end 128.4765 88.086498) (width 0.5) (layer B.Cu) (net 7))
 (segment (start 135.023001 75.741157) (end 130.894001 79.870157) (width 0.5) (layer B.Cu) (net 7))
 (segment (start 135.023001 73.510001) (end 135.023001 75.741157) (width 0.5) (layer B.Cu) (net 7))
 (segment (start 130.894001 79.870157) (end 130.894001 85.668997) (width 0.5) (layer B.Cu) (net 7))
 (segment (start 128.4765 88.086498) (end 128.4765 88.5165) (width 0.5) (layer B.Cu) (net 7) (status 20))
 (segment (start 130.4765 87.5665) (end 130.5265 87.5665) (width 0.5) (layer B.Cu) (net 6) (status 30))
 (via (at 133.477 79.6925) (size 0.8) (drill 0.4) (layers F.Cu B.Cu) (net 6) (status 30))
 (segment (start 131.494012 86.548988) (end 131.494012 81.675488) (width 0.5) (layer B.Cu) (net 6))
 (segment (start 130.4765 87.5665) (end 131.494012 86.548988) (width 0.5) (layer B.Cu) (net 6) (status 10))
 (segment (start 131.494012 81.675488) (end 133.477 79.6925) (width 0.5) (layer B.Cu) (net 6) (status 20)))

